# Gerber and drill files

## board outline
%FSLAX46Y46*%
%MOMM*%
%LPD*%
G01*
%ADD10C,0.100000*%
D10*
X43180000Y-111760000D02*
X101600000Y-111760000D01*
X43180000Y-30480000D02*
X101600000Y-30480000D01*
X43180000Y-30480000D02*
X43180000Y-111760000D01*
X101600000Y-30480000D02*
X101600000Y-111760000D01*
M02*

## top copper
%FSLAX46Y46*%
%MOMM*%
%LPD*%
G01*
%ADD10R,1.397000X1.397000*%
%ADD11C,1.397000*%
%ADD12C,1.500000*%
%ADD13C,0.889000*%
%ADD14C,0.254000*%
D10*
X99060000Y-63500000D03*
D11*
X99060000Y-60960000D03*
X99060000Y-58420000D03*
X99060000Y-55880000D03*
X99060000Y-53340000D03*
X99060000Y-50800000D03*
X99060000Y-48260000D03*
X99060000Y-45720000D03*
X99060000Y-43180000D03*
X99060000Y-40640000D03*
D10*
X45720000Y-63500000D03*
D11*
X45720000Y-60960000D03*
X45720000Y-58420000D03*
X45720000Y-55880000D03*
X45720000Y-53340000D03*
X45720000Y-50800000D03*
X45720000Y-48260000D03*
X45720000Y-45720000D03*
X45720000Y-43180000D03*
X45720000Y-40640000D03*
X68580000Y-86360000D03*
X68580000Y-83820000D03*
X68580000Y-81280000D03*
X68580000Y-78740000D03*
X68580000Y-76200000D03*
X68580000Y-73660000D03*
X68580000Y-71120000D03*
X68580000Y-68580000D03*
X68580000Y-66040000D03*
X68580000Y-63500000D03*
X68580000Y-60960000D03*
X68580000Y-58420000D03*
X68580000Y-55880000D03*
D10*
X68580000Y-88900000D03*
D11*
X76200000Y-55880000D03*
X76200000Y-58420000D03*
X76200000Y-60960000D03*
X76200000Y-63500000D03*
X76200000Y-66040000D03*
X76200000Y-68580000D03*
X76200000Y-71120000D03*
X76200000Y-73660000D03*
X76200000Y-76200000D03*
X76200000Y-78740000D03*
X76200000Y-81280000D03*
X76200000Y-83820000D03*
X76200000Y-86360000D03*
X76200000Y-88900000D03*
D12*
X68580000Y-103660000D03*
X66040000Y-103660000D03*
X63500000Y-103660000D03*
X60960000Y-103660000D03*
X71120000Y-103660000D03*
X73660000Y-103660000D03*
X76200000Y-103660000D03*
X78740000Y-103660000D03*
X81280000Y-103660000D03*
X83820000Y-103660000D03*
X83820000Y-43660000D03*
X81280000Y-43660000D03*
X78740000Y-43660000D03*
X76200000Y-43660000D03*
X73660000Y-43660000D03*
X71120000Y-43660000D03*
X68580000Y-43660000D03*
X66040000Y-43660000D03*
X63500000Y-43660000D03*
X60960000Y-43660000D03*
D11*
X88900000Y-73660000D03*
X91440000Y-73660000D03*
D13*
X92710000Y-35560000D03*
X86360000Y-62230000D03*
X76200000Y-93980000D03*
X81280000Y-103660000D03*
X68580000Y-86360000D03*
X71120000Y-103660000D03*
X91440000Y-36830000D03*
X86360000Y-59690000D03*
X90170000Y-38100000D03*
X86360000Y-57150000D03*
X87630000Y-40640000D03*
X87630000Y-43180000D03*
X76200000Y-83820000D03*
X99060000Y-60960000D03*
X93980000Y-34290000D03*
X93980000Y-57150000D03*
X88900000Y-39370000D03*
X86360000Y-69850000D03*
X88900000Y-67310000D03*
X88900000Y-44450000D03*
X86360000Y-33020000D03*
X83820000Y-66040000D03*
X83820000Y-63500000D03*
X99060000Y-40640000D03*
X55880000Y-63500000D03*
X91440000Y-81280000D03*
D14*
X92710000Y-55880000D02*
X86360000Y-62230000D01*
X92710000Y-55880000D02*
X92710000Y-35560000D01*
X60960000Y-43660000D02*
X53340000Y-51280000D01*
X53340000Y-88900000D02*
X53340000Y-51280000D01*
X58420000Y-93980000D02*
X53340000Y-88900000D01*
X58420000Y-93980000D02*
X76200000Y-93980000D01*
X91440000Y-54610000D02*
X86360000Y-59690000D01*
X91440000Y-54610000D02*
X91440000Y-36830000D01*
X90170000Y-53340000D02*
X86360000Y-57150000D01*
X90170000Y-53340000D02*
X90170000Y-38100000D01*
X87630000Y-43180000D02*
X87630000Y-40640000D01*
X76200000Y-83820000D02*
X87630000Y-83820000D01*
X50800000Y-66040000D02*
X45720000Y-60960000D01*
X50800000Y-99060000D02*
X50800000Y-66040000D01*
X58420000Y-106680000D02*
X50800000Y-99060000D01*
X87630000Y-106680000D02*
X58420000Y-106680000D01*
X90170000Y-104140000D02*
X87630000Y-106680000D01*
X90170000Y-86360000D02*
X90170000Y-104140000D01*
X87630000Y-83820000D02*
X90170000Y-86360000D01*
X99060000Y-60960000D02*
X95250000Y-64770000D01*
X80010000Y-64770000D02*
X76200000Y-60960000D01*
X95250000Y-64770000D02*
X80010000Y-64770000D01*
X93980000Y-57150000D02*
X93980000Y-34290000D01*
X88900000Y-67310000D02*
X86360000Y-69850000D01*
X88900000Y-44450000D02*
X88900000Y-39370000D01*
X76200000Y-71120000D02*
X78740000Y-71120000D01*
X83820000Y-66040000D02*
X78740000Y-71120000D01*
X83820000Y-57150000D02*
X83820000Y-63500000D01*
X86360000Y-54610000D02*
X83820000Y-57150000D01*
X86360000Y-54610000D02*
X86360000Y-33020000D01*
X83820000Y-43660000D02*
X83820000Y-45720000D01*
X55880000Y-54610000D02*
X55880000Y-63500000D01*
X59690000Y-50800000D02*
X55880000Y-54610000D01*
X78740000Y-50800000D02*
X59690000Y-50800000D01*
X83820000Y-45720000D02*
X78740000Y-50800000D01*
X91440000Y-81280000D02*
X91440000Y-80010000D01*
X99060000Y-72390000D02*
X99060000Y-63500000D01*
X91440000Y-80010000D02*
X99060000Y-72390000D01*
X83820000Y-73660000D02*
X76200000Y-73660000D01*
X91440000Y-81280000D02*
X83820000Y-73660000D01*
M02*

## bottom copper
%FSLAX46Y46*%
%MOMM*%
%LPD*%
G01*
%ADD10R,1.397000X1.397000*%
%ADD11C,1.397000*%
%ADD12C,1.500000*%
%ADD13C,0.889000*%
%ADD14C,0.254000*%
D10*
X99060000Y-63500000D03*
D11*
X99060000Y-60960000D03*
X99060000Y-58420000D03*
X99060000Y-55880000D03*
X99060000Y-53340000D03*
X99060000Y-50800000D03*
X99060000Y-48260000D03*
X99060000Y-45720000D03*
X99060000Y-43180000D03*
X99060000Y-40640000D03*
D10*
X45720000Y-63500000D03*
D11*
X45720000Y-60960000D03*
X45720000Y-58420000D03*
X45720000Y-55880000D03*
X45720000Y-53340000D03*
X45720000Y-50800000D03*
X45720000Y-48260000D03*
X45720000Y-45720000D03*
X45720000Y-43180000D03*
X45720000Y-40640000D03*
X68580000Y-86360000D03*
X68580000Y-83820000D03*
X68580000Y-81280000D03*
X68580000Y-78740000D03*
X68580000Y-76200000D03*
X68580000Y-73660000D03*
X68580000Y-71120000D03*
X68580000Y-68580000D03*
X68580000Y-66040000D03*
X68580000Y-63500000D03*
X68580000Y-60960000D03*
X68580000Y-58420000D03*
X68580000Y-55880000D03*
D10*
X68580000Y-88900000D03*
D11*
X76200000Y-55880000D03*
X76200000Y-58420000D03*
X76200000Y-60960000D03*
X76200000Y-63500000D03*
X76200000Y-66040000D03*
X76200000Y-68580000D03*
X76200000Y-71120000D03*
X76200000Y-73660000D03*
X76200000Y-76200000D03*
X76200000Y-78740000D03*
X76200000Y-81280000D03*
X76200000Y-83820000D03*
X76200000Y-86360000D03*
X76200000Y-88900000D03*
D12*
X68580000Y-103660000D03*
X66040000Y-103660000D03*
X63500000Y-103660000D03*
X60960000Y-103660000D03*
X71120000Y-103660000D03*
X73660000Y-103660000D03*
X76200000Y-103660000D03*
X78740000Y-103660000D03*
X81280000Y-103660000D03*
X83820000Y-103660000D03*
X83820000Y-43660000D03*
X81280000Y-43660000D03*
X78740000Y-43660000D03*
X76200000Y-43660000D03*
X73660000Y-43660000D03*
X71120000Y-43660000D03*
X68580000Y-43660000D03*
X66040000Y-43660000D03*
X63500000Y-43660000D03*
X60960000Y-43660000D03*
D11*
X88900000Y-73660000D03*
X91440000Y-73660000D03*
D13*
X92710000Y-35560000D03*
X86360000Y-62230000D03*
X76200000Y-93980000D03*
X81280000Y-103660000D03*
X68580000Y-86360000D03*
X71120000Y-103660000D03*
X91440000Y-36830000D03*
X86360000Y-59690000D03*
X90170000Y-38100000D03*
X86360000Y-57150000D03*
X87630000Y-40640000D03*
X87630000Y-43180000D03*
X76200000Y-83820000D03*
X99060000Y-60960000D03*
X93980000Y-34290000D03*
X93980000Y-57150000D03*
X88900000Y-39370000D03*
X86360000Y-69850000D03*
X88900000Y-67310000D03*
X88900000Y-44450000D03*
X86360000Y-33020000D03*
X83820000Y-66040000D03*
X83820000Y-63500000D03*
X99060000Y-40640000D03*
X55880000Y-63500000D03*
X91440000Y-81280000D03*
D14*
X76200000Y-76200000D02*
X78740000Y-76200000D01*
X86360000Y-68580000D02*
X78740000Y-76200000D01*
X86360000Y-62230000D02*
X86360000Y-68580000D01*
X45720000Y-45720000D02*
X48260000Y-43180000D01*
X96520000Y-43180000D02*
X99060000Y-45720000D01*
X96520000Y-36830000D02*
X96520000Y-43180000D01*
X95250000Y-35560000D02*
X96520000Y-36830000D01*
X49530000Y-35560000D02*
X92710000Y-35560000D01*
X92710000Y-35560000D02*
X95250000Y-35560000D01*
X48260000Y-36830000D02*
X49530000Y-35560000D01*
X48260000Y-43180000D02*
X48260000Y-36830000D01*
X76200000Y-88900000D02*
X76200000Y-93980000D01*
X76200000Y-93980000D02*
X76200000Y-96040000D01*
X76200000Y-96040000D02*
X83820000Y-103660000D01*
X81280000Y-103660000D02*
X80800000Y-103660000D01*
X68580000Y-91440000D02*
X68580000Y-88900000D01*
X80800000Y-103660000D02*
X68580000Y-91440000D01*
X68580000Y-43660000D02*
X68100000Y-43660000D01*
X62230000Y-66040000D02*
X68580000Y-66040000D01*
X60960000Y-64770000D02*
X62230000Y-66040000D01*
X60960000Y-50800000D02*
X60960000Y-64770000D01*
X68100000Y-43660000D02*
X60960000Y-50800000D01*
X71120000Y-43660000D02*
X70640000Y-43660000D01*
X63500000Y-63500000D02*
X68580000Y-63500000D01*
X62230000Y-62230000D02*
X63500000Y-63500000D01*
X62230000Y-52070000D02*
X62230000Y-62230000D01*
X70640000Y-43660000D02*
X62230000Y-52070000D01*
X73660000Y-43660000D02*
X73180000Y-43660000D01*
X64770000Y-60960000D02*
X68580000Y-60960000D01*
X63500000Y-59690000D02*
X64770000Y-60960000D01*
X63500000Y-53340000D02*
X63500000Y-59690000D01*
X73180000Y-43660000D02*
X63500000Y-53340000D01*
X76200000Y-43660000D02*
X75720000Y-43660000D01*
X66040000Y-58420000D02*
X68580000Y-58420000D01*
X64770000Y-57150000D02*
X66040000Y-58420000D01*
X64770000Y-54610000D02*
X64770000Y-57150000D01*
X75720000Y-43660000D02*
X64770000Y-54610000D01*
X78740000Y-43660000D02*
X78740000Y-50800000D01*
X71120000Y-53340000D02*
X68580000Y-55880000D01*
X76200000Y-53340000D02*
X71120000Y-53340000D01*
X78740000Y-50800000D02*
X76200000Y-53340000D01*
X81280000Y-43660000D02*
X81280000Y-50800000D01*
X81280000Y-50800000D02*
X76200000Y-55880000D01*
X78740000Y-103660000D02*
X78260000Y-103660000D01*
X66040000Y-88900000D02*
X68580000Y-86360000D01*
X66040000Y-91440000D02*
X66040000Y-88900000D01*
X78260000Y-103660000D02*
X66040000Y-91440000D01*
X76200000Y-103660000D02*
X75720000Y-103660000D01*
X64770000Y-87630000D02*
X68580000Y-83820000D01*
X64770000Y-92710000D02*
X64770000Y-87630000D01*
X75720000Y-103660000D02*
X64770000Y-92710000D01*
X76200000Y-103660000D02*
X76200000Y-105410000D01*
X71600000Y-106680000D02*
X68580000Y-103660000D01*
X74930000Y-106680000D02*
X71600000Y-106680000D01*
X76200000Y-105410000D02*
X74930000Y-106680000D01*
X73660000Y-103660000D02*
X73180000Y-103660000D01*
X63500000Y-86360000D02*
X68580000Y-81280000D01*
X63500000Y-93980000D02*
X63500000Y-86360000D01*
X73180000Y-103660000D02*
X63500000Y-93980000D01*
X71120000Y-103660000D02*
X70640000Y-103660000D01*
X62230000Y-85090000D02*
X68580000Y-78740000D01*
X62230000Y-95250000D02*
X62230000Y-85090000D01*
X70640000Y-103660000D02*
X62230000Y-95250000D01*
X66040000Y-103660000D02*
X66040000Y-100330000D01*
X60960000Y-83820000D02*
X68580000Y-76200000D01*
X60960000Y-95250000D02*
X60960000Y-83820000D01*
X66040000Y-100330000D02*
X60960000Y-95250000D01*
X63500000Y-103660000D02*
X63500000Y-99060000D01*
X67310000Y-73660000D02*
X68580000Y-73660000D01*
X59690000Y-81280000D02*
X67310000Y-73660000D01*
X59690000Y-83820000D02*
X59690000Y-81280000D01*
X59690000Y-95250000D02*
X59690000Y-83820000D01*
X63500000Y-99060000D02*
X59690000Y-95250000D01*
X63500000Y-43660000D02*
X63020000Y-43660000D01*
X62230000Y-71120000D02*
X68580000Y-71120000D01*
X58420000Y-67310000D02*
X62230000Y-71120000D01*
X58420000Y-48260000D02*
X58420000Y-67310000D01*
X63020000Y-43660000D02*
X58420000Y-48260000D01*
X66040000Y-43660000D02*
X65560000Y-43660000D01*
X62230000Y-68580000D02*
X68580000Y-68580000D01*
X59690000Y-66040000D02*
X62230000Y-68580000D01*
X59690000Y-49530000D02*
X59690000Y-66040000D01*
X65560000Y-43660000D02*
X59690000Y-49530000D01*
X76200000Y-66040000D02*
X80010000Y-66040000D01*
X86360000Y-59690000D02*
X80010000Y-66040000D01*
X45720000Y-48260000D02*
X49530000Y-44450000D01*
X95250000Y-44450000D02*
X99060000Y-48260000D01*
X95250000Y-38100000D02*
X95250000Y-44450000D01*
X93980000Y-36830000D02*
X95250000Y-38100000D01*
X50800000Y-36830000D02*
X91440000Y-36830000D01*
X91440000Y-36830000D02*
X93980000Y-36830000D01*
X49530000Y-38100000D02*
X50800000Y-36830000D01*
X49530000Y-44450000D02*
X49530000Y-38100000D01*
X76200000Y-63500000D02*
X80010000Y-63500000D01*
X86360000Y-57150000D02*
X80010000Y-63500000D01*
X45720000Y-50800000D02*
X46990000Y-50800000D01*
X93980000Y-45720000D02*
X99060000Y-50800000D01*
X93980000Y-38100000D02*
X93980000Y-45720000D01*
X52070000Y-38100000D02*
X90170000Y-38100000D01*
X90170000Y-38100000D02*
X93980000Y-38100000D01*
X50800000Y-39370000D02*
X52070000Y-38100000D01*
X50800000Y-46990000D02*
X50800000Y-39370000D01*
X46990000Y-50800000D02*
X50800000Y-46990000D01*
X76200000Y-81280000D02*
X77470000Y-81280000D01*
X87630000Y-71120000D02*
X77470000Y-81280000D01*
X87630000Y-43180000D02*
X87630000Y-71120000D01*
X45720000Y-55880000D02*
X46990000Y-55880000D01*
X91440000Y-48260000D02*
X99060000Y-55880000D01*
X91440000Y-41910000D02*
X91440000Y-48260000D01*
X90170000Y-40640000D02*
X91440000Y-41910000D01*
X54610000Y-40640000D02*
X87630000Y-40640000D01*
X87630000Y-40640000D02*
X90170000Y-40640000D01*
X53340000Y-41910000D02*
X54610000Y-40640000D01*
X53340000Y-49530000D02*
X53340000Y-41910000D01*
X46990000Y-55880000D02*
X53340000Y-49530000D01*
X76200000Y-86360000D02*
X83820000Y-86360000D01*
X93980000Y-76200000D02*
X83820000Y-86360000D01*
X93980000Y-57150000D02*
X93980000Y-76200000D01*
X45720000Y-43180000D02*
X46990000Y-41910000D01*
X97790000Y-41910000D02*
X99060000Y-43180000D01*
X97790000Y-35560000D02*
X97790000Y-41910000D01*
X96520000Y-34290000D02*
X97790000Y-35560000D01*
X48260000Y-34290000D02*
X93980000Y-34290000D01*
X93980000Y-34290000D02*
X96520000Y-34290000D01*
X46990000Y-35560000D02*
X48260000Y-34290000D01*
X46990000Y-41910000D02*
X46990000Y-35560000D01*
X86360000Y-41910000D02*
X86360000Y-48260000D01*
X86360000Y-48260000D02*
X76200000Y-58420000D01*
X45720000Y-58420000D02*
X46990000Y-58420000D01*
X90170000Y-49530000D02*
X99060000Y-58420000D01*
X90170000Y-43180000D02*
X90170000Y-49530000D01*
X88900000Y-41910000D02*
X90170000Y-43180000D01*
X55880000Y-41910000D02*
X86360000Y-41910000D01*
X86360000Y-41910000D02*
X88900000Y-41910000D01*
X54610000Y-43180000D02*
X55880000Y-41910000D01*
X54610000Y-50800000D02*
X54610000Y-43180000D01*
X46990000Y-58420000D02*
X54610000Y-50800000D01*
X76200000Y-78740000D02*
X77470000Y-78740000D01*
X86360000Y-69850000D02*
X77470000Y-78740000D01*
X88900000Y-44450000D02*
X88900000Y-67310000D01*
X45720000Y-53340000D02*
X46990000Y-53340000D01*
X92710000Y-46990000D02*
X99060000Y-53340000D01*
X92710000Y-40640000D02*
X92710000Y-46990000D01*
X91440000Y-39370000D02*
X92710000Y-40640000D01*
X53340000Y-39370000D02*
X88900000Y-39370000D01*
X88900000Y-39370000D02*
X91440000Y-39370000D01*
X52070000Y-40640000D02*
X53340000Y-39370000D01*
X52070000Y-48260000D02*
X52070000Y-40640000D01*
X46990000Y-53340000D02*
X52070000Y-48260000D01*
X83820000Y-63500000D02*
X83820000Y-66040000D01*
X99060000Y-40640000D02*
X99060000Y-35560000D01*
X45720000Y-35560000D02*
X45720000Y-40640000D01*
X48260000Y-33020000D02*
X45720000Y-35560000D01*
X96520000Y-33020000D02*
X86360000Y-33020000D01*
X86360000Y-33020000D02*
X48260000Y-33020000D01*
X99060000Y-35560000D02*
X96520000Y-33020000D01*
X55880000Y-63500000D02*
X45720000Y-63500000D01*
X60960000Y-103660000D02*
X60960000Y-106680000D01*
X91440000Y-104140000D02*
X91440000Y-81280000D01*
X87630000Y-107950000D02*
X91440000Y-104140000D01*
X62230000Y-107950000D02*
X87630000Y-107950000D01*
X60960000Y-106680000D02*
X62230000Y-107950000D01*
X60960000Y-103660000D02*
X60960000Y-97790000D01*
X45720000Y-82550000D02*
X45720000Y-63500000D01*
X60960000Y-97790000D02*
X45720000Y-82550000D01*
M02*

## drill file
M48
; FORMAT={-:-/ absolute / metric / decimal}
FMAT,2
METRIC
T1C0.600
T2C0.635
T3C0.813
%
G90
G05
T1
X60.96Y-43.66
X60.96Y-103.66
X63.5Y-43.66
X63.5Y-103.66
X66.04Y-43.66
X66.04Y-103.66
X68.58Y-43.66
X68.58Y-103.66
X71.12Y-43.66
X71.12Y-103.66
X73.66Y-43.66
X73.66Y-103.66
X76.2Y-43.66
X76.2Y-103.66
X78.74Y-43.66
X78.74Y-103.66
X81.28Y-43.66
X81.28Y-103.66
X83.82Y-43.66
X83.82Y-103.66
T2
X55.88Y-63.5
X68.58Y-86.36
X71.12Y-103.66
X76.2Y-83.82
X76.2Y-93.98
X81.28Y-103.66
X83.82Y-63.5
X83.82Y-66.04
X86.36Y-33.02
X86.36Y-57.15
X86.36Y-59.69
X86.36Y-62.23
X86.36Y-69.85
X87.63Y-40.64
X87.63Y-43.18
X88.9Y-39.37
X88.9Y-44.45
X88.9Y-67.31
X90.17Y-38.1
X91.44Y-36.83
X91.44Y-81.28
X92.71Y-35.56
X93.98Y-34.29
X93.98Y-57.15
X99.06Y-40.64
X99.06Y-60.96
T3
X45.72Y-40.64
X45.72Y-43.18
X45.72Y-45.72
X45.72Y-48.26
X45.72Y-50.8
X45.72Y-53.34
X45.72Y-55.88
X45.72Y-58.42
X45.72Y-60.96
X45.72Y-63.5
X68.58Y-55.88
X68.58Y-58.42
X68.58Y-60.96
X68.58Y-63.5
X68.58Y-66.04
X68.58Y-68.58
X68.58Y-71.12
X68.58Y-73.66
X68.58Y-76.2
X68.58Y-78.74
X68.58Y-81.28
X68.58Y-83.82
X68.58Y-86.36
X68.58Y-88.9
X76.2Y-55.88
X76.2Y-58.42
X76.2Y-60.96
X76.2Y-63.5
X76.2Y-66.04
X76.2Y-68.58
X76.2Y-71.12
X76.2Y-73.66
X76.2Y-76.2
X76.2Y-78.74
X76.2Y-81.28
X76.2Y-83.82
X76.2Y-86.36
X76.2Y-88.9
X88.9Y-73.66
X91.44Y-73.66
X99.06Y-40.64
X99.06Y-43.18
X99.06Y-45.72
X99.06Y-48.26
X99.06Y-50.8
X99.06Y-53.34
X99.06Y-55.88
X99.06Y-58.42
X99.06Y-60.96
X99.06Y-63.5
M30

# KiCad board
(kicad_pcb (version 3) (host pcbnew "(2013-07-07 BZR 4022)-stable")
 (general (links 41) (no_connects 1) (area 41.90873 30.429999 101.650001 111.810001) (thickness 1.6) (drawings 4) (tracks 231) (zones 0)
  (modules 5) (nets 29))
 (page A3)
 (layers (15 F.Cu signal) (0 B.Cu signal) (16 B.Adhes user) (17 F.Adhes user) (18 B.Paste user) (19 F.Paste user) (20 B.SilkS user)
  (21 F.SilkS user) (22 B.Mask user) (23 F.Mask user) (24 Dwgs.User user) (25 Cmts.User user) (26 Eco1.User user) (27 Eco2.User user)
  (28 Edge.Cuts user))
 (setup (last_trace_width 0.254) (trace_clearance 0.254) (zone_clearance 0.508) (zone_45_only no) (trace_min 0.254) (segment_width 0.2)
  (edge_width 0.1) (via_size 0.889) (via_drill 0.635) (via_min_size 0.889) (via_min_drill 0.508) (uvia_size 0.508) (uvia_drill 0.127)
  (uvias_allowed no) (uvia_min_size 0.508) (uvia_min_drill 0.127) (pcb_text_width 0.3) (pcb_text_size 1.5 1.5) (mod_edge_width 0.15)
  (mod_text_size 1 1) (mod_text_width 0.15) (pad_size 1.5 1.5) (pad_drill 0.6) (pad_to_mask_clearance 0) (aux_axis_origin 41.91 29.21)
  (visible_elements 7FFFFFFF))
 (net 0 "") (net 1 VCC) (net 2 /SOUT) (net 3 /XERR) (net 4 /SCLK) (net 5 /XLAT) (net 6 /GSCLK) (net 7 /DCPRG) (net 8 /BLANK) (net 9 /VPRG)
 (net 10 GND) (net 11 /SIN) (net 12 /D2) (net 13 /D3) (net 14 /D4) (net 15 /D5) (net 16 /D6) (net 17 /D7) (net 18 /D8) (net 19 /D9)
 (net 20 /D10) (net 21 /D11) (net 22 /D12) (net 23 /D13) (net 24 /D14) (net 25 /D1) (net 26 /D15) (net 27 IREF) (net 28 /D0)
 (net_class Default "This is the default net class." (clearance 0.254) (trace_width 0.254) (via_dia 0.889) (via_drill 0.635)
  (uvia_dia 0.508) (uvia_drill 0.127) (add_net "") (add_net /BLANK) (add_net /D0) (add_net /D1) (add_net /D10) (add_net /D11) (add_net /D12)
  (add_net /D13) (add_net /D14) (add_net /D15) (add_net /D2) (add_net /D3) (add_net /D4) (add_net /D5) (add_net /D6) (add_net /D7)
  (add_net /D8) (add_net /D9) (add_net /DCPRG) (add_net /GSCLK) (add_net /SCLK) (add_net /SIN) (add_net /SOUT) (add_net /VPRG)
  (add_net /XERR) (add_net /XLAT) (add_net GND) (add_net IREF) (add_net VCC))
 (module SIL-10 (layer F.Cu) (at 99.06 52.07 90)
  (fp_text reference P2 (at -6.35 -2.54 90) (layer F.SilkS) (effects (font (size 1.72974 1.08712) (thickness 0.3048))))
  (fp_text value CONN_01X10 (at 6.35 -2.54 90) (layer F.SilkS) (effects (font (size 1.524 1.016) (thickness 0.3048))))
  (pad 1 thru_hole rect (at -11.43 0 90) (size 1.397 1.397) (drill 0.8128) (layers *.Cu *.Mask F.SilkS) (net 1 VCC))
  (pad 2 thru_hole circle (at -8.89 0 90) (size 1.397 1.397) (drill 0.8128) (layers *.Cu *.Mask F.SilkS) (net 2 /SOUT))
  (pad 3 thru_hole circle (at -6.35 0 90) (size 1.397 1.397) (drill 0.8128) (layers *.Cu *.Mask F.SilkS) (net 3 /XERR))
  (pad 4 thru_hole circle (at -3.81 0 90) (size 1.397 1.397) (drill 0.8128) (layers *.Cu *.Mask F.SilkS) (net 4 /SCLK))
  (pad 5 thru_hole circle (at -1.27 0 90) (size 1.397 1.397) (drill 0.8128) (layers *.Cu *.Mask F.SilkS) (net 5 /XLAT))
  (pad 6 thru_hole circle (at 1.27 0 90) (size 1.397 1.397) (drill 0.8128) (layers *.Cu *.Mask F.SilkS) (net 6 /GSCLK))
  (pad 7 thru_hole circle (at 3.81 0 90) (size 1.397 1.397) (drill 0.8128) (layers *.Cu *.Mask F.SilkS) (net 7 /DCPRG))
  (pad 8 thru_hole circle (at 6.35 0 90) (size 1.397 1.397) (drill 0.8128) (layers *.Cu *.Mask F.SilkS) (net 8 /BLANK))
  (pad 9 thru_hole circle (at 8.89 0 90) (size 1.397 1.397) (drill 0.8128) (layers *.Cu *.Mask F.SilkS) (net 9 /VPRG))
  (pad 10 thru_hole circle (at 11.43 0 90) (size 1.397 1.397) (drill 0.8128) (layers *.Cu *.Mask F.SilkS) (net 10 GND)))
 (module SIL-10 (layer F.Cu) (at 45.72 52.07 90)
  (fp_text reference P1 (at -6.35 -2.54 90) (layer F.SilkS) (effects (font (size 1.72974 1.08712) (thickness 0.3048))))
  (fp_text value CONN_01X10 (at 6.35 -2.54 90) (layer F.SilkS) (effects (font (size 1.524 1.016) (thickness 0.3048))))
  (pad 1 thru_hole rect (at -11.43 0 90) (size 1.397 1.397) (drill 0.8128) (layers *.Cu *.Mask F.SilkS) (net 1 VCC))
  (pad 2 thru_hole circle (at -8.89 0 90) (size 1.397 1.397) (drill 0.8128) (layers *.Cu *.Mask F.SilkS) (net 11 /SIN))
  (pad 3 thru_hole circle (at -6.35 0 90) (size 1.397 1.397) (drill 0.8128) (layers *.Cu *.Mask F.SilkS) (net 3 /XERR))
  (pad 4 thru_hole circle (at -3.81 0 90) (size 1.397 1.397) (drill 0.8128) (layers *.Cu *.Mask F.SilkS) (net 4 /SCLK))
  (pad 5 thru_hole circle (at -1.27 0 90) (size 1.397 1.397) (drill 0.8128) (layers *.Cu *.Mask F.SilkS) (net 5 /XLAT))
  (pad 6 thru_hole circle (at 1.27 0 90) (size 1.397 1.397) (drill 0.8128) (layers *.Cu *.Mask F.SilkS) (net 6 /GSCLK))
  (pad 7 thru_hole circle (at 3.81 0 90) (size 1.397 1.397) (drill 0.8128) (layers *.Cu *.Mask F.SilkS) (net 7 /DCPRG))
  (pad 8 thru_hole circle (at 6.35 0 90) (size 1.397 1.397) (drill 0.8128) (layers *.Cu *.Mask F.SilkS) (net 8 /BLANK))
  (pad 9 thru_hole circle (at 8.89 0 90) (size 1.397 1.397) (drill 0.8128) (layers *.Cu *.Mask F.SilkS) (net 9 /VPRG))
  (pad 10 thru_hole circle (at 11.43 0 90) (size 1.397 1.397) (drill 0.8128) (layers *.Cu *.Mask F.SilkS) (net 10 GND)))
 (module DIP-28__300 (layer B.Cu) (at 72.39 72.39 90)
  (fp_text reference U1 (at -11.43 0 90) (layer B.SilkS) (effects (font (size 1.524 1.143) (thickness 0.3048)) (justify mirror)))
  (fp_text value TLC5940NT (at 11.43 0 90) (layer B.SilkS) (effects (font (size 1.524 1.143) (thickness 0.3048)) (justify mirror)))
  (pad 2 thru_hole circle (at -13.97 -3.81 90) (size 1.397 1.397) (drill 0.8128) (layers *.Cu *.Mask B.SilkS) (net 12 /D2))
  (pad 3 thru_hole circle (at -11.43 -3.81 90) (size 1.397 1.397) (drill 0.8128) (layers *.Cu *.Mask B.SilkS) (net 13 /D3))
  (pad 4 thru_hole circle (at -8.89 -3.81 90) (size 1.397 1.397) (drill 0.8128) (layers *.Cu *.Mask B.SilkS) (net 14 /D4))
  (pad 5 thru_hole circle (at -6.35 -3.81 90) (size 1.397 1.397) (drill 0.8128) (layers *.Cu *.Mask B.SilkS) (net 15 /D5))
  (pad 6 thru_hole circle (at -3.81 -3.81 90) (size 1.397 1.397) (drill 0.8128) (layers *.Cu *.Mask B.SilkS) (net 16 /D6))
  (pad 7 thru_hole circle (at -1.27 -3.81 90) (size 1.397 1.397) (drill 0.8128) (layers *.Cu *.Mask B.SilkS) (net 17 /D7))
  (pad 8 thru_hole circle (at 1.27 -3.81 90) (size 1.397 1.397) (drill 0.8128) (layers *.Cu *.Mask B.SilkS) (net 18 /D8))
  (pad 9 thru_hole circle (at 3.81 -3.81 90) (size 1.397 1.397) (drill 0.8128) (layers *.Cu *.Mask B.SilkS) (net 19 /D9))
  (pad 10 thru_hole circle (at 6.35 -3.81 90) (size 1.397 1.397) (drill 0.8128) (layers *.Cu *.Mask B.SilkS) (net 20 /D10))
  (pad 11 thru_hole circle (at 8.89 -3.81 90) (size 1.397 1.397) (drill 0.8128) (layers *.Cu *.Mask B.SilkS) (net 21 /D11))
  (pad 12 thru_hole circle (at 11.43 -3.81 90) (size 1.397 1.397) (drill 0.8128) (layers *.Cu *.Mask B.SilkS) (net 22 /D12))
  (pad 13 thru_hole circle (at 13.97 -3.81 90) (size 1.397 1.397) (drill 0.8128) (layers *.Cu *.Mask B.SilkS) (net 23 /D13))
  (pad 14 thru_hole circle (at 16.51 -3.81 90) (size 1.397 1.397) (drill 0.8128) (layers *.Cu *.Mask B.SilkS) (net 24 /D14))
  (pad 1 thru_hole rect (at -16.51 -3.81 90) (size 1.397 1.397) (drill 0.8128) (layers *.Cu *.Mask B.SilkS) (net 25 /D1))
  (pad 15 thru_hole circle (at 16.51 3.81 90) (size 1.397 1.397) (drill 0.8128) (layers *.Cu *.Mask B.SilkS) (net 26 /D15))
  (pad 16 thru_hole circle (at 13.97 3.81 90) (size 1.397 1.397) (drill 0.8128) (layers *.Cu *.Mask B.SilkS) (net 3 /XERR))
  (pad 17 thru_hole circle (at 11.43 3.81 90) (size 1.397 1.397) (drill 0.8128) (layers *.Cu *.Mask B.SilkS) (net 2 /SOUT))
  (pad 18 thru_hole circle (at 8.89 3.81 90) (size 1.397 1.397) (drill 0.8128) (layers *.Cu *.Mask B.SilkS) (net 6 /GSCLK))
  (pad 19 thru_hole circle (at 6.35 3.81 90) (size 1.397 1.397) (drill 0.8128) (layers *.Cu *.Mask B.SilkS) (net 7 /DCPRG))
  (pad 20 thru_hole circle (at 3.81 3.81 90) (size 1.397 1.397) (drill 0.8128) (layers *.Cu *.Mask B.SilkS) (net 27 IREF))
  (pad 21 thru_hole circle (at 1.27 3.81 90) (size 1.397 1.397) (drill 0.8128) (layers *.Cu *.Mask B.SilkS) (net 10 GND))
  (pad 22 thru_hole circle (at -1.27 3.81 90) (size 1.397 1.397) (drill 0.8128) (layers *.Cu *.Mask B.SilkS) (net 1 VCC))
  (pad 23 thru_hole circle (at -3.81 3.81 90) (size 1.397 1.397) (drill 0.8128) (layers *.Cu *.Mask B.SilkS) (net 8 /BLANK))
  (pad 24 thru_hole circle (at -6.35 3.81 90) (size 1.397 1.397) (drill 0.8128) (layers *.Cu *.Mask B.SilkS) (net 5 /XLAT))
  (pad 25 thru_hole circle (at -8.89 3.81 90) (size 1.397 1.397) (drill 0.8128) (layers *.Cu *.Mask B.SilkS) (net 4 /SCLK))
  (pad 26 thru_hole circle (at -11.43 3.81 90) (size 1.397 1.397) (drill 0.8128) (layers *.Cu *.Mask B.SilkS) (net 11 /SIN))
  (pad 27 thru_hole circle (at -13.97 3.81 90) (size 1.397 1.397) (drill 0.8128) (layers *.Cu *.Mask B.SilkS) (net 9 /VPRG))
  (pad 28 thru_hole circle (at -16.51 3.81 90) (size 1.397 1.397) (drill 0.8128) (layers *.Cu *.Mask B.SilkS) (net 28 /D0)))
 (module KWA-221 (layer F.Cu) (at 72.39 73.66)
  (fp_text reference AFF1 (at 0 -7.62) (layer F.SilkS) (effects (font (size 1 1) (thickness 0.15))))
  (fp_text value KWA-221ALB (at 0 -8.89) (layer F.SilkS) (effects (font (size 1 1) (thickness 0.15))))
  (pad 4 thru_hole circle (at -3.81 30) (size 1.5 1.5) (drill 0.6) (layers *.Cu *.Mask F.SilkS) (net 13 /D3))
  (pad 3 thru_hole circle (at -6.35 30) (size 1.5 1.5) (drill 0.6) (layers *.Cu *.Mask F.SilkS) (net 16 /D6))
  (pad 2 thru_hole circle (at -8.89 30) (size 1.5 1.5) (drill 0.6) (layers *.Cu *.Mask F.SilkS) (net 17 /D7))
  (pad 1 thru_hole circle (at -11.43 30) (size 1.5 1.5) (drill 0.6) (layers *.Cu *.Mask F.SilkS) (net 1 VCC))
  (pad 5 thru_hole circle (at -1.27 30) (size 1.5 1.5) (drill 0.6) (layers *.Cu *.Mask F.SilkS) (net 15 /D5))
  (pad 6 thru_hole circle (at 1.27 30) (size 1.5 1.5) (drill 0.6) (layers *.Cu *.Mask F.SilkS) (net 14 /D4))
  (pad 7 thru_hole circle (at 3.81 30) (size 1.5 1.5) (drill 0.6) (layers *.Cu *.Mask F.SilkS) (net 13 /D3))
  (pad 8 thru_hole circle (at 6.35 30) (size 1.5 1.5) (drill 0.6) (layers *.Cu *.Mask F.SilkS) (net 12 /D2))
  (pad 9 thru_hole circle (at 8.89 30) (size 1.5 1.5) (drill 0.6) (layers *.Cu *.Mask F.SilkS) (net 25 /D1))
  (pad 10 thru_hole circle (at 11.43 30) (size 1.5 1.5) (drill 0.6) (layers *.Cu *.Mask F.SilkS) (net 28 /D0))
  (pad 11 thru_hole circle (at 11.43 -30) (size 1.5 1.5) (drill 0.6) (layers *.Cu *.Mask F.SilkS) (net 1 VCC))
  (pad 12 thru_hole circle (at 8.89 -30) (size 1.5 1.5) (drill 0.6) (layers *.Cu *.Mask F.SilkS) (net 26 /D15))
  (pad 13 thru_hole circle (at 6.35 -30) (size 1.5 1.5) (drill 0.6) (layers *.Cu *.Mask F.SilkS) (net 24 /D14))
  (pad 14 thru_hole circle (at 3.81 -30) (size 1.5 1.5) (drill 0.6) (layers *.Cu *.Mask F.SilkS) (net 23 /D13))
  (pad 15 thru_hole circle (at 1.27 -30) (size 1.5 1.5) (drill 0.6) (layers *.Cu *.Mask F.SilkS) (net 22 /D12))
  (pad 16 thru_hole circle (at -1.27 -30) (size 1.5 1.5) (drill 0.6) (layers *.Cu *.Mask F.SilkS) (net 21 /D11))
  (pad 17 thru_hole circle (at -3.81 -30) (size 1.5 1.5) (drill 0.6) (layers *.Cu *.Mask F.SilkS) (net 20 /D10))
  (pad 18 thru_hole circle (at -6.35 -30) (size 1.5 1.5) (drill 0.6) (layers *.Cu *.Mask F.SilkS) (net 19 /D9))
  (pad 19 thru_hole circle (at -8.89 -30) (size 1.5 1.5) (drill 0.6) (layers *.Cu *.Mask F.SilkS) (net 18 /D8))
  (pad 20 thru_hole circle (at -11.43 -30) (size 1.5 1.5) (drill 0.6) (layers *.Cu *.Mask F.SilkS) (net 28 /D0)))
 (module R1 (layer B.Cu) (at 90.17 73.66) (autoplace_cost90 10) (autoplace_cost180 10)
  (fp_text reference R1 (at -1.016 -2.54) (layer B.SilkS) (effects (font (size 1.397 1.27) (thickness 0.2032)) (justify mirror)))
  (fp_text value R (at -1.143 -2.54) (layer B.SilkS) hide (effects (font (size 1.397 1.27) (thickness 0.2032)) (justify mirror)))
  (pad 1 thru_hole circle (at -1.27 0) (size 1.397 1.397) (drill 0.8128) (layers *.Cu *.Mask B.SilkS) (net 27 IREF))
  (pad 2 thru_hole circle (at 1.27 0) (size 1.397 1.397) (drill 0.8128) (layers *.Cu *.Mask B.SilkS)))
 (gr_line (start 43.18 111.76) (end 101.6 111.76) (angle 90) (layer Edge.Cuts) (width 0.1))
 (gr_line (start 43.18 30.48) (end 101.6 30.48) (angle 90) (layer Edge.Cuts) (width 0.1))
 (gr_line (start 43.18 30.48) (end 43.18 111.76) (angle 90) (layer Edge.Cuts) (width 0.1))
 (gr_line (start 101.6 30.48) (end 101.6 111.76) (angle 90) (layer Edge.Cuts) (width 0.1))
 (via (at 92.71 35.56) (size 0.889) (layers F.Cu B.Cu) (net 8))
 (segment (start 76.2 76.2) (end 78.74 76.2) (width 0.254) (layer B.Cu) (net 8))
 (segment (start 86.36 68.58) (end 78.74 76.2) (width 0.254) (layer B.Cu) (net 8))
 (segment (start 86.36 62.23) (end 86.36 68.58) (width 0.254) (layer B.Cu) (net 8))
 (via (at 86.36 62.23) (size 0.889) (layers F.Cu B.Cu) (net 8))
 (segment (start 92.71 55.88) (end 86.36 62.23) (width 0.254) (layer F.Cu) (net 8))
 (segment (start 92.71 55.88) (end 92.71 35.56) (width 0.254) (layer F.Cu) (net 8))
 (segment (start 45.72 45.72) (end 48.26 43.18) (width 0.254) (layer B.Cu) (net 8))
 (segment (start 96.52 43.18) (end 99.06 45.72) (width 0.254) (layer B.Cu) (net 8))
 (segment (start 96.52 36.83) (end 96.52 43.18) (width 0.254) (layer B.Cu) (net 8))
 (segment (start 95.25 35.56) (end 96.52 36.83) (width 0.254) (layer B.Cu) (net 8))
 (segment (start 49.53 35.56) (end 92.71 35.56) (width 0.254) (layer B.Cu) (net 8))
 (segment (start 92.71 35.56) (end 95.25 35.56) (width 0.254) (layer B.Cu) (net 8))
 (segment (start 48.26 36.83) (end 49.53 35.56) (width 0.254) (layer B.Cu) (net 8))
 (segment (start 48.26 43.18) (end 48.26 36.83) (width 0.254) (layer B.Cu) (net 8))
 (via (at 76.2 93.98) (size 0.889) (layers F.Cu B.Cu) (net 28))
 (segment (start 60.96 43.66) (end 53.34 51.28) (width 0.254) (layer F.Cu) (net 28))
 (segment (start 53.34 88.9) (end 53.34 51.28) (width 0.254) (layer F.Cu) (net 28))
 (segment (start 58.42 93.98) (end 53.34 88.9) (width 0.254) (layer F.Cu) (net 28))
 (segment (start 58.42 93.98) (end 76.2 93.98) (width 0.254) (layer F.Cu) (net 28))
 (segment (start 76.2 88.9) (end 76.2 93.98) (width 0.254) (layer B.Cu) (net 28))
 (segment (start 76.2 93.98) (end 76.2 96.04) (width 0.254) (layer B.Cu) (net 28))
 (segment (start 76.2 96.04) (end 83.82 103.66) (width 0.254) (layer B.Cu) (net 28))
 (segment (start 81.28 103.66) (end 80.8 103.66) (width 0.254) (layer B.Cu) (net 25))
 (segment (start 68.58 91.44) (end 68.58 88.9) (width 0.254) (layer B.Cu) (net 25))
 (segment (start 80.8 103.66) (end 68.58 91.44) (width 0.254) (layer B.Cu) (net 25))
 (via (at 81.28 103.66) (size 0.889) (layers F.Cu B.Cu) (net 25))
 (segment (start 68.58 43.66) (end 68.1 43.66) (width 0.254) (layer B.Cu) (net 20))
 (segment (start 62.23 66.04) (end 68.58 66.04) (width 0.254) (layer B.Cu) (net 20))
 (segment (start 60.96 64.77) (end 62.23 66.04) (width 0.254) (layer B.Cu) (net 20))
 (segment (start 60.96 50.8) (end 60.96 64.77) (width 0.254) (layer B.Cu) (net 20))
 (segment (start 68.1 43.66) (end 60.96 50.8) (width 0.254) (layer B.Cu) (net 20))
 (segment (start 71.12 43.66) (end 70.64 43.66) (width 0.254) (layer B.Cu) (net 21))
 (segment (start 63.5 63.5) (end 68.58 63.5) (width 0.254) (layer B.Cu) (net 21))
 (segment (start 62.23 62.23) (end 63.5 63.5) (width 0.254) (layer B.Cu) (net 21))
 (segment (start 62.23 52.07) (end 62.23 62.23) (width 0.254) (layer B.Cu) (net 21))
 (segment (start 70.64 43.66) (end 62.23 52.07) (width 0.254) (layer B.Cu) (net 21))
 (segment (start 73.66 43.66) (end 73.18 43.66) (width 0.254) (layer B.Cu) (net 22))
 (segment (start 64.77 60.96) (end 68.58 60.96) (width 0.254) (layer B.Cu) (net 22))
 (segment (start 63.5 59.69) (end 64.77 60.96) (width 0.254) (layer B.Cu) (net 22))
 (segment (start 63.5 53.34) (end 63.5 59.69) (width 0.254) (layer B.Cu) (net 22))
 (segment (start 73.18 43.66) (end 63.5 53.34) (width 0.254) (layer B.Cu) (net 22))
 (segment (start 76.2 43.66) (end 75.72 43.66) (width 0.254) (layer B.Cu) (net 23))
 (segment (start 66.04 58.42) (end 68.58 58.42) (width 0.254) (layer B.Cu) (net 23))
 (segment (start 64.77 57.15) (end 66.04 58.42) (width 0.254) (layer B.Cu) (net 23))
 (segment (start 64.77 54.61) (end 64.77 57.15) (width 0.254) (layer B.Cu) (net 23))
 (segment (start 75.72 43.66) (end 64.77 54.61) (width 0.254) (layer B.Cu) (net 23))
 (segment (start 78.74 43.66) (end 78.74 50.8) (width 0.254) (layer B.Cu) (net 24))
 (segment (start 71.12 53.34) (end 68.58 55.88) (width 0.254) (layer B.Cu) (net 24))
 (segment (start 76.2 53.34) (end 71.12 53.34) (width 0.254) (layer B.Cu) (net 24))
 (segment (start 78.74 50.8) (end 76.2 53.34) (width 0.254) (layer B.Cu) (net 24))
 (segment (start 81.28 43.66) (end 81.28 50.8) (width 0.254) (layer B.Cu) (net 26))
 (segment (start 81.28 50.8) (end 76.2 55.88) (width 0.254) (layer B.Cu) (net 26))
 (segment (start 78.74 103.66) (end 78.26 103.66) (width 0.254) (layer B.Cu) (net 12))
 (segment (start 66.04 88.9) (end 68.58 86.36) (width 0.254) (layer B.Cu) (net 12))
 (segment (start 66.04 91.44) (end 66.04 88.9) (width 0.254) (layer B.Cu) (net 12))
 (segment (start 78.26 103.66) (end 66.04 91.44) (width 0.254) (layer B.Cu) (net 12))
 (via (at 68.58 86.36) (size 0.889) (layers F.Cu B.Cu) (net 12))
 (segment (start 76.2 103.66) (end 75.72 103.66) (width 0.254) (layer B.Cu) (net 13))
 (segment (start 64.77 87.63) (end 68.58 83.82) (width 0.254) (layer B.Cu) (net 13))
 (segment (start 64.77 92.71) (end 64.77 87.63) (width 0.254) (layer B.Cu) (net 13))
 (segment (start 75.72 103.66) (end 64.77 92.71) (width 0.254) (layer B.Cu) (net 13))
 (segment (start 76.2 103.66) (end 76.2 105.41) (width 0.254) (layer B.Cu) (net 13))
 (segment (start 71.6 106.68) (end 68.58 103.66) (width 0.254) (layer B.Cu) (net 13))
 (segment (start 74.93 106.68) (end 71.6 106.68) (width 0.254) (layer B.Cu) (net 13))
 (segment (start 76.2 105.41) (end 74.93 106.68) (width 0.254) (layer B.Cu) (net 13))
 (segment (start 73.66 103.66) (end 73.18 103.66) (width 0.254) (layer B.Cu) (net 14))
 (segment (start 63.5 86.36) (end 68.58 81.28) (width 0.254) (layer B.Cu) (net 14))
 (segment (start 63.5 93.98) (end 63.5 86.36) (width 0.254) (layer B.Cu) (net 14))
 (segment (start 73.18 103.66) (end 63.5 93.98) (width 0.254) (layer B.Cu) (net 14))
 (segment (start 71.12 103.66) (end 70.64 103.66) (width 0.254) (layer B.Cu) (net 15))
 (segment (start 62.23 85.09) (end 68.58 78.74) (width 0.254) (layer B.Cu) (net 15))
 (segment (start 62.23 95.25) (end 62.23 85.09) (width 0.254) (layer B.Cu) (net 15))
 (segment (start 70.64 103.66) (end 62.23 95.25) (width 0.254) (layer B.Cu) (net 15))
 (via (at 71.12 103.66) (size 0.889) (layers F.Cu B.Cu) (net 15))
 (segment (start 66.04 103.66) (end 66.04 100.33) (width 0.254) (layer B.Cu) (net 16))
 (segment (start 60.96 83.82) (end 68.58 76.2) (width 0.254) (layer B.Cu) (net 16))
 (segment (start 60.96 95.25) (end 60.96 83.82) (width 0.254) (layer B.Cu) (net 16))
 (segment (start 66.04 100.33) (end 60.96 95.25) (width 0.254) (layer B.Cu) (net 16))
 (segment (start 63.5 103.66) (end 63.5 99.06) (width 0.254) (layer B.Cu) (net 17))
 (segment (start 67.31 73.66) (end 68.58 73.66) (width 0.254) (layer B.Cu) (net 17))
 (segment (start 59.69 81.28) (end 67.31 73.66) (width 0.254) (layer B.Cu) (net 17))
 (segment (start 59.69 83.82) (end 59.69 81.28) (width 0.254) (layer B.Cu) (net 17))
 (segment (start 59.69 95.25) (end 59.69 83.82) (width 0.254) (layer B.Cu) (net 17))
 (segment (start 63.5 99.06) (end 59.69 95.25) (width 0.254) (layer B.Cu) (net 17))
 (segment (start 63.5 43.66) (end 63.02 43.66) (width 0.254) (layer B.Cu) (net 18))
 (segment (start 62.23 71.12) (end 68.58 71.12) (width 0.254) (layer B.Cu) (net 18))
 (segment (start 58.42 67.31) (end 62.23 71.12) (width 0.254) (layer B.Cu) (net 18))
 (segment (start 58.42 48.26) (end 58.42 67.31) (width 0.254) (layer B.Cu) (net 18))
 (segment (start 63.02 43.66) (end 58.42 48.26) (width 0.254) (layer B.Cu) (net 18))
 (segment (start 66.04 43.66) (end 65.56 43.66) (width 0.254) (layer B.Cu) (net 19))
 (segment (start 62.23 68.58) (end 68.58 68.58) (width 0.254) (layer B.Cu) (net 19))
 (segment (start 59.69 66.04) (end 62.23 68.58) (width 0.254) (layer B.Cu) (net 19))
 (segment (start 59.69 49.53) (end 59.69 66.04) (width 0.254) (layer B.Cu) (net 19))
 (segment (start 65.56 43.66) (end 59.69 49.53) (width 0.254) (layer B.Cu) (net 19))
 (via (at 91.44 36.83) (size 0.889) (layers F.Cu B.Cu) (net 7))
 (segment (start 76.2 66.04) (end 80.01 66.04) (width 0.254) (layer B.Cu) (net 7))
 (segment (start 86.36 59.69) (end 80.01 66.04) (width 0.254) (layer B.Cu) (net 7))
 (via (at 86.36 59.69) (size 0.889) (layers F.Cu B.Cu) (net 7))
 (segment (start 91.44 54.61) (end 86.36 59.69) (width 0.254) (layer F.Cu) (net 7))
 (segment (start 91.44 54.61) (end 91.44 36.83) (width 0.254) (layer F.Cu) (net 7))
 (segment (start 45.72 48.26) (end 49.53 44.45) (width 0.254) (layer B.Cu) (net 7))
 (segment (start 95.25 44.45) (end 99.06 48.26) (width 0.254) (layer B.Cu) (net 7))
 (segment (start 95.25 38.1) (end 95.25 44.45) (width 0.254) (layer B.Cu) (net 7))
 (segment (start 93.98 36.83) (end 95.25 38.1) (width 0.254) (layer B.Cu) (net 7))
 (segment (start 50.8 36.83) (end 91.44 36.83) (width 0.254) (layer B.Cu) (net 7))
 (segment (start 91.44 36.83) (end 93.98 36.83) (width 0.254) (layer B.Cu) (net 7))
 (segment (start 49.53 38.1) (end 50.8 36.83) (width 0.254) (layer B.Cu) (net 7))
 (segment (start 49.53 44.45) (end 49.53 38.1) (width 0.254) (layer B.Cu) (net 7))
 (via (at 90.17 38.1) (size 0.889) (layers F.Cu B.Cu) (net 6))
 (segment (start 76.2 63.5) (end 80.01 63.5) (width 0.254) (layer B.Cu) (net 6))
 (segment (start 86.36 57.15) (end 80.01 63.5) (width 0.254) (layer B.Cu) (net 6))
 (via (at 86.36 57.15) (size 0.889) (layers F.Cu B.Cu) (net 6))
 (segment (start 90.17 53.34) (end 86.36 57.15) (width 0.254) (layer F.Cu) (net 6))
 (segment (start 90.17 53.34) (end 90.17 38.1) (width 0.254) (layer F.Cu) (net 6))
 (segment (start 45.72 50.8) (end 46.99 50.8) (width 0.254) (layer B.Cu) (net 6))
 (segment (start 93.98 45.72) (end 99.06 50.8) (width 0.254) (layer B.Cu) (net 6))
 (segment (start 93.98 38.1) (end 93.98 45.72) (width 0.254) (layer B.Cu) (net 6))
 (segment (start 52.07 38.1) (end 90.17 38.1) (width 0.254) (layer B.Cu) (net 6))
 (segment (start 90.17 38.1) (end 93.98 38.1) (width 0.254) (layer B.Cu) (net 6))
 (segment (start 50.8 39.37) (end 52.07 38.1) (width 0.254) (layer B.Cu) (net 6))
 (segment (start 50.8 46.99) (end 50.8 39.37) (width 0.254) (layer B.Cu) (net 6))
 (segment (start 46.99 50.8) (end 50.8 46.99) (width 0.254) (layer B.Cu) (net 6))
 (via (at 87.63 40.64) (size 0.889) (layers F.Cu B.Cu) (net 4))
 (segment (start 76.2 81.28) (end 77.47 81.28) (width 0.254) (layer B.Cu) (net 4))
 (segment (start 87.63 71.12) (end 77.47 81.28) (width 0.254) (layer B.Cu) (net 4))
 (segment (start 87.63 43.18) (end 87.63 71.12) (width 0.254) (layer B.Cu) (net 4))
 (via (at 87.63 43.18) (size 0.889) (layers F.Cu B.Cu) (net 4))
 (segment (start 87.63 43.18) (end 87.63 40.64) (width 0.254) (layer F.Cu) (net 4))
 (segment (start 45.72 55.88) (end 46.99 55.88) (width 0.254) (layer B.Cu) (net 4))
 (segment (start 91.44 48.26) (end 99.06 55.88) (width 0.254) (layer B.Cu) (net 4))
 (segment (start 91.44 41.91) (end 91.44 48.26) (width 0.254) (layer B.Cu) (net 4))
 (segment (start 90.17 40.64) (end 91.44 41.91) (width 0.254) (layer B.Cu) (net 4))
 (segment (start 54.61 40.64) (end 87.63 40.64) (width 0.254) (layer B.Cu) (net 4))
 (segment (start 87.63 40.64) (end 90.17 40.64) (width 0.254) (layer B.Cu) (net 4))
 (segment (start 53.34 41.91) (end 54.61 40.64) (width 0.254) (layer B.Cu) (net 4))
 (segment (start 53.34 49.53) (end 53.34 41.91) (width 0.254) (layer B.Cu) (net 4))
 (segment (start 46.99 55.88) (end 53.34 49.53) (width 0.254) (layer B.Cu) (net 4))
 (via (at 76.2 83.82) (size 0.889) (layers F.Cu B.Cu) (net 11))
 (segment (start 76.2 83.82) (end 87.63 83.82) (width 0.254) (layer F.Cu) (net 11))
 (segment (start 50.8 66.04) (end 45.72 60.96) (width 0.254) (layer F.Cu) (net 11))
 (segment (start 50.8 99.06) (end 50.8 66.04) (width 0.254) (layer F.Cu) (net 11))
 (segment (start 58.42 106.68) (end 50.8 99.06) (width 0.254) (layer F.Cu) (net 11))
 (segment (start 87.63 106.68) (end 58.42 106.68) (width 0.254) (layer F.Cu) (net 11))
 (segment (start 90.17 104.14) (end 87.63 106.68) (width 0.254) (layer F.Cu) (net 11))
 (segment (start 90.17 86.36) (end 90.17 104.14) (width 0.254) (layer F.Cu) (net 11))
 (segment (start 87.63 83.82) (end 90.17 86.36) (width 0.254) (layer F.Cu) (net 11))
 (via (at 99.06 60.96) (size 0.889) (layers F.Cu B.Cu) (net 2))
 (segment (start 99.06 60.96) (end 95.25 64.77) (width 0.254) (layer F.Cu) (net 2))
 (segment (start 80.01 64.77) (end 76.2 60.96) (width 0.254) (layer F.Cu) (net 2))
 (segment (start 95.25 64.77) (end 80.01 64.77) (width 0.254) (layer F.Cu) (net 2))
 (via (at 93.98 34.29) (size 0.889) (layers F.Cu B.Cu) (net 9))
 (segment (start 76.2 86.36) (end 83.82 86.36) (width 0.254) (layer B.Cu) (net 9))
 (segment (start 93.98 76.2) (end 83.82 86.36) (width 0.254) (layer B.Cu) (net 9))
 (segment (start 93.98 57.15) (end 93.98 76.2) (width 0.254) (layer B.Cu) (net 9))
 (via (at 93.98 57.15) (size 0.889) (layers F.Cu B.Cu) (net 9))
 (segment (start 93.98 57.15) (end 93.98 34.29) (width 0.254) (layer F.Cu) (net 9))
 (segment (start 45.72 43.18) (end 46.99 41.91) (width 0.254) (layer B.Cu) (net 9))
 (segment (start 97.79 41.91) (end 99.06 43.18) (width 0.254) (layer B.Cu) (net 9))
 (segment (start 97.79 35.56) (end 97.79 41.91) (width 0.254) (layer B.Cu) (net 9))
 (segment (start 96.52 34.29) (end 97.79 35.56) (width 0.254) (layer B.Cu) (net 9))
 (segment (start 48.26 34.29) (end 93.98 34.29) (width 0.254) (layer B.Cu) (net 9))
 (segment (start 93.98 34.29) (end 96.52 34.29) (width 0.254) (layer B.Cu) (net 9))
 (segment (start 46.99 35.56) (end 48.26 34.29) (width 0.254) (layer B.Cu) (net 9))
 (segment (start 46.99 41.91) (end 46.99 35.56) (width 0.254) (layer B.Cu) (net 9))
 (segment (start 86.36 41.91) (end 86.36 48.26) (width 0.254) (layer B.Cu) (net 3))
 (segment (start 86.36 48.26) (end 76.2 58.42) (width 0.254) (layer B.Cu) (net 3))
 (segment (start 45.72 58.42) (end 46.99 58.42) (width 0.254) (layer B.Cu) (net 3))
 (segment (start 90.17 49.53) (end 99.06 58.42) (width 0.254) (layer B.Cu) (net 3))
 (segment (start 90.17 43.18) (end 90.17 49.53) (width 0.254) (layer B.Cu) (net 3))
 (segment (start 88.9 41.91) (end 90.17 43.18) (width 0.254) (layer B.Cu) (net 3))
 (segment (start 55.88 41.91) (end 86.36 41.91) (width 0.254) (layer B.Cu) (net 3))
 (segment (start 86.36 41.91) (end 88.9 41.91) (width 0.254) (layer B.Cu) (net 3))
 (segment (start 54.61 43.18) (end 55.88 41.91) (width 0.254) (layer B.Cu) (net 3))
 (segment (start 54.61 50.8) (end 54.61 43.18) (width 0.254) (layer B.Cu) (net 3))
 (segment (start 46.99 58.42) (end 54.61 50.8) (width 0.254) (layer B.Cu) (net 3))
 (via (at 88.9 39.37) (size 0.889) (layers F.Cu B.Cu) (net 5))
 (segment (start 76.2 78.74) (end 77.47 78.74) (width 0.254) (layer B.Cu) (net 5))
 (segment (start 86.36 69.85) (end 77.47 78.74) (width 0.254) (layer B.Cu) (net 5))
 (via (at 86.36 69.85) (size 0.889) (layers F.Cu B.Cu) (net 5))
 (segment (start 88.9 67.31) (end 86.36 69.85) (width 0.254) (layer F.Cu) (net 5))
 (via (at 88.9 67.31) (size 0.889) (layers F.Cu B.Cu) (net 5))
 (segment (start 88.9 44.45) (end 88.9 67.31) (width 0.254) (layer B.Cu) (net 5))
 (via (at 88.9 44.45) (size 0.889) (layers F.Cu B.Cu) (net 5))
 (segment (start 88.9 44.45) (end 88.9 39.37) (width 0.254) (layer F.Cu) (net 5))
 (segment (start 45.72 53.34) (end 46.99 53.34) (width 0.254) (layer B.Cu) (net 5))
 (segment (start 92.71 46.99) (end 99.06 53.34) (width 0.254) (layer B.Cu) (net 5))
 (segment (start 92.71 40.64) (end 92.71 46.99) (width 0.254) (layer B.Cu) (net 5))
 (segment (start 91.44 39.37) (end 92.71 40.64) (width 0.254) (layer B.Cu) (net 5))
 (segment (start 53.34 39.37) (end 88.9 39.37) (width 0.254) (layer B.Cu) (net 5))
 (segment (start 88.9 39.37) (end 91.44 39.37) (width 0.254) (layer B.Cu) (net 5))
 (segment (start 52.07 40.64) (end 53.34 39.37) (width 0.254) (layer B.Cu) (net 5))
 (segment (start 52.07 48.26) (end 52.07 40.64) (width 0.254) (layer B.Cu) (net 5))
 (segment (start 46.99 53.34) (end 52.07 48.26) (width 0.254) (layer B.Cu) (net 5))
 (via (at 86.36 33.02) (size 0.889) (layers F.Cu B.Cu) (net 10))
 (segment (start 76.2 71.12) (end 78.74 71.12) (width 0.254) (layer F.Cu) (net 10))
 (segment (start 83.82 66.04) (end 78.74 71.12) (width 0.254) (layer F.Cu) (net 10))
 (via (at 83.82 66.04) (size 0.889) (layers F.Cu B.Cu) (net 10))
 (segment (start 83.82 63.5) (end 83.82 66.04) (width 0.254) (layer B.Cu) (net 10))
 (via (at 83.82 63.5) (size 0.889) (layers F.Cu B.Cu) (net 10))
 (segment (start 83.82 57.15) (end 83.82 63.5) (width 0.254) (layer F.Cu) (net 10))
 (segment (start 86.36 54.61) (end 83.82 57.15) (width 0.254) (layer F.Cu) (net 10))
 (segment (start 86.36 54.61) (end 86.36 33.02) (width 0.254) (layer F.Cu) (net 10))
 (via (at 99.06 40.64) (size 0.889) (layers F.Cu B.Cu) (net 10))
 (segment (start 99.06 40.64) (end 99.06 35.56) (width 0.254) (layer B.Cu) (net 10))
 (segment (start 45.72 35.56) (end 45.72 40.64) (width 0.254) (layer B.Cu) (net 10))
 (segment (start 48.26 33.02) (end 45.72 35.56) (width 0.254) (layer B.Cu) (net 10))
 (segment (start 96.52 33.02) (end 86.36 33.02) (width 0.254) (layer B.Cu) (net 10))
 (segment (start 86.36 33.02) (end 48.26 33.02) (width 0.254) (layer B.Cu) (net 10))
 (segment (start 99.06 35.56) (end 96.52 33.02) (width 0.254) (layer B.Cu) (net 10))
 (segment (start 83.82 43.66) (end 83.82 45.72) (width 0.254) (layer F.Cu) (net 1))
 (segment (start 55.88 63.5) (end 45.72 63.5) (width 0.254) (layer B.Cu) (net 1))
 (via (at 55.88 63.5) (size 0.889) (layers F.Cu B.Cu) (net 1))
 (segment (start 55.88 54.61) (end 55.88 63.5) (width 0.254) (layer F.Cu) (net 1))
 (segment (start 59.69 50.8) (end 55.88 54.61) (width 0.254) (layer F.Cu) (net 1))
 (segment (start 78.74 50.8) (end 59.69 50.8) (width 0.254) (layer F.Cu) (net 1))
 (segment (start 83.82 45.72) (end 78.74 50.8) (width 0.254) (layer F.Cu) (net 1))
 (segment (start 91.44 81.28) (end 91.44 80.01) (width 0.254) (layer F.Cu) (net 1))
 (segment (start 99.06 72.39) (end 99.06 63.5) (width 0.254) (layer F.Cu) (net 1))
 (segment (start 91.44 80.01) (end 99.06 72.39) (width 0.254) (layer F.Cu) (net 1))
 (segment (start 60.96 103.66) (end 60.96 106.68) (width 0.254) (layer B.Cu) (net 1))
 (segment (start 83.82 73.66) (end 76.2 73.66) (width 0.254) (layer F.Cu) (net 1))
 (segment (start 91.44 81.28) (end 83.82 73.66) (width 0.254) (layer F.Cu) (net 1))
 (via (at 91.44 81.28) (size 0.889) (layers F.Cu B.Cu) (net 1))
 (segment (start 91.44 104.14) (end 91.44 81.28) (width 0.254) (layer B.Cu) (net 1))
 (segment (start 87.63 107.95) (end 91.44 104.14) (width 0.254) (layer B.Cu) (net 1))
 (segment (start 62.23 107.95) (end 87.63 107.95) (width 0.254) (layer B.Cu) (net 1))
 (segment (start 60.96 106.68) (end 62.23 107.95) (width 0.254) (layer B.Cu) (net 1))
 (segment (start 60.96 103.66) (end 60.96 97.79) (width 0.254) (layer B.Cu) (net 1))
 (segment (start 45.72 82.55) (end 45.72 63.5) (width 0.254) (layer B.Cu) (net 1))
 (segment (start 60.96 97.79) (end 45.72 82.55) (width 0.254) (layer B.Cu) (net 1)))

